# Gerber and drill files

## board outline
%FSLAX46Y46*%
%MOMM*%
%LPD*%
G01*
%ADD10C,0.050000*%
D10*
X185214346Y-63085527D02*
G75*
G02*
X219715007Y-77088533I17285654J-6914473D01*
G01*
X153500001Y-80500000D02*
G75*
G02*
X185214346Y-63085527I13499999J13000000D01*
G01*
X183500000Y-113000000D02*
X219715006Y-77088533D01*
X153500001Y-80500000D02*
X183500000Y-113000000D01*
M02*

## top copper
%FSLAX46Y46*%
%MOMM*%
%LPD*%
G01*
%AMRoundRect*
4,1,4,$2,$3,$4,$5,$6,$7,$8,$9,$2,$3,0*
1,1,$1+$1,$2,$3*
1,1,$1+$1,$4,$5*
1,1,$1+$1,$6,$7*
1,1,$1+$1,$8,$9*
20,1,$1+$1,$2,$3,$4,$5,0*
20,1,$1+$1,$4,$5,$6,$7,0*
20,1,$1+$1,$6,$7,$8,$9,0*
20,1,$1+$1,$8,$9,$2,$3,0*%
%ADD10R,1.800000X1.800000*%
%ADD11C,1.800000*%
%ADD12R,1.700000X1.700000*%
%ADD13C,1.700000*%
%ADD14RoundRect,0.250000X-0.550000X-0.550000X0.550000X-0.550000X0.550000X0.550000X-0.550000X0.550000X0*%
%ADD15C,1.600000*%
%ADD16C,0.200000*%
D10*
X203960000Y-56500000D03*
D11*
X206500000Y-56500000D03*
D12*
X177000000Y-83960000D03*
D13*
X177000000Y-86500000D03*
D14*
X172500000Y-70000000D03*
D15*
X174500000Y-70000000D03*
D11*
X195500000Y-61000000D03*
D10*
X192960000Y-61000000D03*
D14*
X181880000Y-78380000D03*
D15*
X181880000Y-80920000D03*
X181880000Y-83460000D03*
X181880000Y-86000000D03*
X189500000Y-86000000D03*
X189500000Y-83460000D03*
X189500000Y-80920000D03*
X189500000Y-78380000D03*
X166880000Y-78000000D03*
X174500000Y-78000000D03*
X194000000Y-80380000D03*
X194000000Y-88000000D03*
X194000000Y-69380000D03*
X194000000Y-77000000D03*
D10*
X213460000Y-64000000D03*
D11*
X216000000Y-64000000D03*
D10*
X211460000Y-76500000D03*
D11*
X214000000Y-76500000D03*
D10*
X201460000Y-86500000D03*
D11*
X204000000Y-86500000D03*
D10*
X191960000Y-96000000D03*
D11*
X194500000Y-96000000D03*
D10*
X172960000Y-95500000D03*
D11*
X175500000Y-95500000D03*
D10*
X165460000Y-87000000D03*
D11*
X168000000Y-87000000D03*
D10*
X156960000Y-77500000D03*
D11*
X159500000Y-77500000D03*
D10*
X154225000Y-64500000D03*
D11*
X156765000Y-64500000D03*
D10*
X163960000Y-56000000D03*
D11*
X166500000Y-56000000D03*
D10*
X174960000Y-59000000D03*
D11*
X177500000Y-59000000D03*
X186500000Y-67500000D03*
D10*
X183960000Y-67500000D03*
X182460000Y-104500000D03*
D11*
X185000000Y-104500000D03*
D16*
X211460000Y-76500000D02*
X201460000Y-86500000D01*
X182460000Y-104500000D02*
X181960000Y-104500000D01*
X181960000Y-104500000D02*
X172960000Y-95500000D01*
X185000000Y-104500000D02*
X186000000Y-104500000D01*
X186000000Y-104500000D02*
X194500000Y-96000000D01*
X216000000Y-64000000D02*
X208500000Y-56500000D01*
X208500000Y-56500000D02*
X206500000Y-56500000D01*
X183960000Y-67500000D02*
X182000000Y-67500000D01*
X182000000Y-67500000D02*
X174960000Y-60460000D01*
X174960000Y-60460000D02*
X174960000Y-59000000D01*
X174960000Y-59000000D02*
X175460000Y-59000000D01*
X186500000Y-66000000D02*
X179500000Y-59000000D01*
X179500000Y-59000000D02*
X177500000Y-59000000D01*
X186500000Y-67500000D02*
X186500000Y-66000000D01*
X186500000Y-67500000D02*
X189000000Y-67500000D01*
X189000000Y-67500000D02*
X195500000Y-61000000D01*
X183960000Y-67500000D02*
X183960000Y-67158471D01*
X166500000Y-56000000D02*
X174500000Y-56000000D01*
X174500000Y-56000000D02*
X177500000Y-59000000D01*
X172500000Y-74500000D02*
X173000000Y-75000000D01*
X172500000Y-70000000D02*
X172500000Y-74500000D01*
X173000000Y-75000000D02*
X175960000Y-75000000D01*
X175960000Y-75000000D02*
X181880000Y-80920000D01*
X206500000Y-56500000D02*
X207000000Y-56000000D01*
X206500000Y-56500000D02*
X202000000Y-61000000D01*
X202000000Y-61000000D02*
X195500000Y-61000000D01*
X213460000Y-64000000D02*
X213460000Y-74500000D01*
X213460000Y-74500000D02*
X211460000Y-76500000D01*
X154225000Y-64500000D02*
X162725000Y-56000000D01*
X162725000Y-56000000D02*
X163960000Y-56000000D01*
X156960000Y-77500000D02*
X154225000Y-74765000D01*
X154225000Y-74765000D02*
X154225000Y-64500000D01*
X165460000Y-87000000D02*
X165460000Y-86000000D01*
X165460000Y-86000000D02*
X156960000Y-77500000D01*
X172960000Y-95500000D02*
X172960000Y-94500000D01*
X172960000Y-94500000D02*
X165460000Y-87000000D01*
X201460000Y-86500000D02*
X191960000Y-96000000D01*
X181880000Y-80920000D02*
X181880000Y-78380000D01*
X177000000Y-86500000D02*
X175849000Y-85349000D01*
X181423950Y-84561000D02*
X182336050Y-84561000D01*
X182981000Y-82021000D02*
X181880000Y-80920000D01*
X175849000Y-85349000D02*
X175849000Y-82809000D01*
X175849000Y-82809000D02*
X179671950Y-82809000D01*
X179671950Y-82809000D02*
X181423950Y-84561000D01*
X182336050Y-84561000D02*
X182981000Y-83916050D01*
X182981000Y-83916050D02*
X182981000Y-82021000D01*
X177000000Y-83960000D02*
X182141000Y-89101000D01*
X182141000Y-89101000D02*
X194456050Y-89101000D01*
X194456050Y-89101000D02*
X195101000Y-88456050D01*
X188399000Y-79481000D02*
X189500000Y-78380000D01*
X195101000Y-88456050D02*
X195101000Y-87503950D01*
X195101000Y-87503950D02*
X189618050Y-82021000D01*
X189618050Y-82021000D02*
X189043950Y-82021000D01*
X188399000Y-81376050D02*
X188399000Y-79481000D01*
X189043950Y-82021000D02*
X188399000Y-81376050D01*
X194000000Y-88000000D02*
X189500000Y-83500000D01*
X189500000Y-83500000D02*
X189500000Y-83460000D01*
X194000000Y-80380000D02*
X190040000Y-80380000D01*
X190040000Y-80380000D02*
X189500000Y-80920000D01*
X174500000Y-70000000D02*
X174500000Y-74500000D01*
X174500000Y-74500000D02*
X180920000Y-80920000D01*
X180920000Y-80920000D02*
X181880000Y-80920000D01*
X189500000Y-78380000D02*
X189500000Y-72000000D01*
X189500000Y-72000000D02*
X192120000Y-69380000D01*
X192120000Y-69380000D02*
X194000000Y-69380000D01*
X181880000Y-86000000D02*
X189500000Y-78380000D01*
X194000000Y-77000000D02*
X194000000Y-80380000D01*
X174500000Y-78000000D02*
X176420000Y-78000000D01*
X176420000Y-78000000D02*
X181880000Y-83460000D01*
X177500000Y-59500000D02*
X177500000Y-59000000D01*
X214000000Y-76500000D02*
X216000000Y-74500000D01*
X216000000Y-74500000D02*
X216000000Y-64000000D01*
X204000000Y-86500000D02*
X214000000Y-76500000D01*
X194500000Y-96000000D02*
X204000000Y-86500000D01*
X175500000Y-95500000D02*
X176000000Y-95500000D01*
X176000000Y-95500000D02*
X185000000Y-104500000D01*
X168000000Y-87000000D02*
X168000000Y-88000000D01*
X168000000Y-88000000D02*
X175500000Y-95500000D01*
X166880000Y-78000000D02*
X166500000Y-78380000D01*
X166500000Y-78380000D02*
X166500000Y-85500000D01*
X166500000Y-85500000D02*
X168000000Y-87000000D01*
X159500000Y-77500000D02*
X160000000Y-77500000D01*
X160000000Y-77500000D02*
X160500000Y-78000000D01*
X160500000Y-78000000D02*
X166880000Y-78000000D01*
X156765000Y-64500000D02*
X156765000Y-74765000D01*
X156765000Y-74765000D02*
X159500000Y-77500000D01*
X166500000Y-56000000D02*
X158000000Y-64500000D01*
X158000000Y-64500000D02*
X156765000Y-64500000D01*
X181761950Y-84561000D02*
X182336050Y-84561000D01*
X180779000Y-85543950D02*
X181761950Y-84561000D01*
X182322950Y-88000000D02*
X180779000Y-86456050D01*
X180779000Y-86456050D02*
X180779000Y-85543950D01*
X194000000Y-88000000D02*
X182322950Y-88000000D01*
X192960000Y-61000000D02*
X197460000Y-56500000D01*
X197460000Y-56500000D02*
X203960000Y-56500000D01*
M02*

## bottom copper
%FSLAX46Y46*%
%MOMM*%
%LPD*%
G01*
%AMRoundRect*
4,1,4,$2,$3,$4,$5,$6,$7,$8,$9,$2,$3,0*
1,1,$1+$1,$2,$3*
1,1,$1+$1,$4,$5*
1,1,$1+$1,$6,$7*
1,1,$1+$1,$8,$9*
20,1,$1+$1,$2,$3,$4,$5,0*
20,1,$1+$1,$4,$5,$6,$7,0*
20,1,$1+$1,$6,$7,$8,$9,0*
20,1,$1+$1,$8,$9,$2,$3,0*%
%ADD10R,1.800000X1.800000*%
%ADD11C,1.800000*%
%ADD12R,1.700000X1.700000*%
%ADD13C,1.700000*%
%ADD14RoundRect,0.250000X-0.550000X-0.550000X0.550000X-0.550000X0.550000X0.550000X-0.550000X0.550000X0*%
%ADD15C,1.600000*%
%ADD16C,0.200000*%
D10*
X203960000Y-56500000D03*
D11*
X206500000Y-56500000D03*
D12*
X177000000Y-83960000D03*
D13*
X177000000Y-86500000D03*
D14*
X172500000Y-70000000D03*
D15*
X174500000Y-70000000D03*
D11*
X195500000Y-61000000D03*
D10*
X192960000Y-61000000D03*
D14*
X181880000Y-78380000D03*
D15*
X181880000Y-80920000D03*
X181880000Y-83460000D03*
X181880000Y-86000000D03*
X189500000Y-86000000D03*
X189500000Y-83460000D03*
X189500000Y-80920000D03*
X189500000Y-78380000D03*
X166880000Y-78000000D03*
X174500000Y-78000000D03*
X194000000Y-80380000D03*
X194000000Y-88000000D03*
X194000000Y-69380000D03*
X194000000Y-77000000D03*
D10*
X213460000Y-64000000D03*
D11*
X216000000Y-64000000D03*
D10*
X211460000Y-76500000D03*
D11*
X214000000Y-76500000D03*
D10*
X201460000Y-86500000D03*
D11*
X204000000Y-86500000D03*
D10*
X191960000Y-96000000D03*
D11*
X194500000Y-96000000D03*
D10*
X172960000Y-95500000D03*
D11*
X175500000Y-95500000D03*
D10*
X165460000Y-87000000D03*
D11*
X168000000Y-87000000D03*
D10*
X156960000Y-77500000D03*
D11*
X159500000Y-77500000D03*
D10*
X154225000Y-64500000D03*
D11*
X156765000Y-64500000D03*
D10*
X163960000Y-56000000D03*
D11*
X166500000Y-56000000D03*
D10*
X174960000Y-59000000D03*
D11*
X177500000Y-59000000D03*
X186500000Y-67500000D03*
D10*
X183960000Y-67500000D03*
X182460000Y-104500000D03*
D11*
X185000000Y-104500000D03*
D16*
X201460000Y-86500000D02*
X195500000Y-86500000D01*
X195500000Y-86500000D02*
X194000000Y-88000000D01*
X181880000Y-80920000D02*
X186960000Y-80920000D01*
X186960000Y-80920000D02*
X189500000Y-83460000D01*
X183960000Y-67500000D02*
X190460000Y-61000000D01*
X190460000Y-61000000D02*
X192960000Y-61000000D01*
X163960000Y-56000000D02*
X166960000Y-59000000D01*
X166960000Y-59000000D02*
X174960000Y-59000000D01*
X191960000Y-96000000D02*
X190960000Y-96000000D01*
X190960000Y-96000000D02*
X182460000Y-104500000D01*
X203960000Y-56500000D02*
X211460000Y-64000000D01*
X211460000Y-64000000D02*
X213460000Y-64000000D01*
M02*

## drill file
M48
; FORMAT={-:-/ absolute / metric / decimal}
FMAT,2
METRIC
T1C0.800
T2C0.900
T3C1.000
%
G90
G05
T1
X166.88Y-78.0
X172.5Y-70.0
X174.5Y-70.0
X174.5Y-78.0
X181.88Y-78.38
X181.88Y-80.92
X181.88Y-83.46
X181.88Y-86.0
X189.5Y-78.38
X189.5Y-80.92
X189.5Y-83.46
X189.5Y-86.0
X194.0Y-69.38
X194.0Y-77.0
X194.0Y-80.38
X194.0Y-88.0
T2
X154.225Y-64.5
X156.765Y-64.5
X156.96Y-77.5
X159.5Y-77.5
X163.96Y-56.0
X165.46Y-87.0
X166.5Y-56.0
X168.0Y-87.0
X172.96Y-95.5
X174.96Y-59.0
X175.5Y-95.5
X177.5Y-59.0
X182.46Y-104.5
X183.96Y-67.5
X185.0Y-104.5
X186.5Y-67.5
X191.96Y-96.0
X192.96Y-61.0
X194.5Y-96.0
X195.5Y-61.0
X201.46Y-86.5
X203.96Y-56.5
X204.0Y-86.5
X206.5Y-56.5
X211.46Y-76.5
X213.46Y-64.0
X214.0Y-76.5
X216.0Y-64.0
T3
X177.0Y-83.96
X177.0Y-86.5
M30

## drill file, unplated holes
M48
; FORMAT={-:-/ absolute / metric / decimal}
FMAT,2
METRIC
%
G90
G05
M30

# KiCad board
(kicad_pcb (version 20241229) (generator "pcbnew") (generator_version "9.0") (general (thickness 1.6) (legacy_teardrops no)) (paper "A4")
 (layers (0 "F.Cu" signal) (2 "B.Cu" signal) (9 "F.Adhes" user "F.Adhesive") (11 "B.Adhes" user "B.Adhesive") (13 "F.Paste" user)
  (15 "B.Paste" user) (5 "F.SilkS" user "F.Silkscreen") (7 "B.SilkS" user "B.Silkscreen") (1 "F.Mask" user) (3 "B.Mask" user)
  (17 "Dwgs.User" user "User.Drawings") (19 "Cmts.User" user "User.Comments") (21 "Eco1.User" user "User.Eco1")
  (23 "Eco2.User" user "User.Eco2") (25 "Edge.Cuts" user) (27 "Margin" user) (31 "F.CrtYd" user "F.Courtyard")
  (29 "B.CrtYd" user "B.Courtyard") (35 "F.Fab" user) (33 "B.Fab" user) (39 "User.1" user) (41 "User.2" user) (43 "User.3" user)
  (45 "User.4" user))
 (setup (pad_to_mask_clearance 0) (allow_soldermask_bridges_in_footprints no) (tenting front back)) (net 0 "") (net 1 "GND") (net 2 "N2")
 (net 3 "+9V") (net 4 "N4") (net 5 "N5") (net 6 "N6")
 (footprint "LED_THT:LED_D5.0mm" (layer "F.Cu") (at 183.96 67.5)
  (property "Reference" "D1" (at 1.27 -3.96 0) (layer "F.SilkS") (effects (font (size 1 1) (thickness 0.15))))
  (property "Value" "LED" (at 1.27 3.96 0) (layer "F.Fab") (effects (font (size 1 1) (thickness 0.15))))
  (pad "1" thru_hole rect (at 0 0) (size 1.8 1.8) (drill 0.9) (layers "*.Cu" "*.Mask") (remove_unused_layers no) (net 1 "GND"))
  (pad "2" thru_hole circle (at 2.54 0) (size 1.8 1.8) (drill 0.9) (layers "*.Cu" "*.Mask") (remove_unused_layers no) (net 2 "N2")))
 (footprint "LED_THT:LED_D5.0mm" (layer "F.Cu") (at 192.96 61)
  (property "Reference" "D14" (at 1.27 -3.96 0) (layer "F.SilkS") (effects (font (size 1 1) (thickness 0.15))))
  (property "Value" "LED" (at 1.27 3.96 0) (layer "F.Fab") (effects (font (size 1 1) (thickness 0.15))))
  (pad "1" thru_hole rect (at 0 0) (size 1.8 1.8) (drill 0.9) (layers "*.Cu" "*.Mask") (remove_unused_layers no) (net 1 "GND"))
  (pad "2" thru_hole circle (at 2.54 0) (size 1.8 1.8) (drill 0.9) (layers "*.Cu" "*.Mask") (remove_unused_layers no) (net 2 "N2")))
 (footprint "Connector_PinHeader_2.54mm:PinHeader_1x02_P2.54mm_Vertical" (layer "F.Cu") (at 177 83.96)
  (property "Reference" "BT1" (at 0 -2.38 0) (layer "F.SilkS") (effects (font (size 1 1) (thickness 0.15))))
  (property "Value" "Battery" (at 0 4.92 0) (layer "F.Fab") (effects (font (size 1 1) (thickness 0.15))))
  (pad "1" thru_hole rect (at 0 0) (size 1.7 1.7) (drill 1) (layers "*.Cu" "*.Mask") (remove_unused_layers no) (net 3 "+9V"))
  (pad "2" thru_hole circle (at 0 2.54) (size 1.7 1.7) (drill 1) (layers "*.Cu" "*.Mask") (remove_unused_layers no) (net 1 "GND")))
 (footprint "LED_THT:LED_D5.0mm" (layer "F.Cu") (at 203.96 56.5)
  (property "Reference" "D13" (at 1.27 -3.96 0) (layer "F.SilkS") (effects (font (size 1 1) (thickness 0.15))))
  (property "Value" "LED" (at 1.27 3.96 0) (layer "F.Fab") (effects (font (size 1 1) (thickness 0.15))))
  (pad "1" thru_hole rect (at 0 0) (size 1.8 1.8) (drill 0.9) (layers "*.Cu" "*.Mask") (remove_unused_layers no) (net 1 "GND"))
  (pad "2" thru_hole circle (at 2.54 0) (size 1.8 1.8) (drill 0.9) (layers "*.Cu" "*.Mask") (remove_unused_layers no) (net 2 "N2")))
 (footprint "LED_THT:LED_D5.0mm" (layer "F.Cu") (at 154.225 64.5)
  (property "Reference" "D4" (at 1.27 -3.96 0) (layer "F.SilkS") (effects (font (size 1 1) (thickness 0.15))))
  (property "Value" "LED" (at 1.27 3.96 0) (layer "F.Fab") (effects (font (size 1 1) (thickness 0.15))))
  (pad "1" thru_hole rect (at 0 0) (size 1.8 1.8) (drill 0.9) (layers "*.Cu" "*.Mask") (remove_unused_layers no) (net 1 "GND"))
  (pad "2" thru_hole circle (at 2.54 0) (size 1.8 1.8) (drill 0.9) (layers "*.Cu" "*.Mask") (remove_unused_layers no) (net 2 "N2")))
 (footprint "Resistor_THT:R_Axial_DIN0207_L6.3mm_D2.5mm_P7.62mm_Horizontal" (layer "F.Cu") (at 166.88 78)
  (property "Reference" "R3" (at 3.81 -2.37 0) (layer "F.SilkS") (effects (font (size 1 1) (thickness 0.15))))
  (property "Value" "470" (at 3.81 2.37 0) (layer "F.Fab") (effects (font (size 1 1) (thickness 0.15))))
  (pad "1" thru_hole circle (at 0 0) (size 1.6 1.6) (drill 0.8) (layers "*.Cu" "*.Mask") (remove_unused_layers no) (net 2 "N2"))
  (pad "2" thru_hole circle (at 7.62 0) (size 1.6 1.6) (drill 0.8) (layers "*.Cu" "*.Mask") (remove_unused_layers no) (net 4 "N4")))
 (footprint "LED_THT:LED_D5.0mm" (layer "F.Cu") (at 172.96 95.5)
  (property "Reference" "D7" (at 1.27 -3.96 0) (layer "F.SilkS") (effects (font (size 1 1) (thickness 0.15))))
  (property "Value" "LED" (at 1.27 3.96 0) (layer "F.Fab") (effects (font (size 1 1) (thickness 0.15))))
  (pad "1" thru_hole rect (at 0 0) (size 1.8 1.8) (drill 0.9) (layers "*.Cu" "*.Mask") (remove_unused_layers no) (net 1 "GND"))
  (pad "2" thru_hole circle (at 2.54 0) (size 1.8 1.8) (drill 0.9) (layers "*.Cu" "*.Mask") (remove_unused_layers no) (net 2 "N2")))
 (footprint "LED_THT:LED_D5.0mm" (layer "F.Cu") (at 191.96 96)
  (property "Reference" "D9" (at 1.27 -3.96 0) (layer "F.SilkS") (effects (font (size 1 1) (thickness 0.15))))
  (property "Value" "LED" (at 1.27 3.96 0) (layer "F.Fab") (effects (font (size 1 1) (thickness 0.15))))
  (pad "1" thru_hole rect (at 0 0) (size 1.8 1.8) (drill 0.9) (layers "*.Cu" "*.Mask") (remove_unused_layers no) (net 1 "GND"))
  (pad "2" thru_hole circle (at 2.54 0) (size 1.8 1.8) (drill 0.9) (layers "*.Cu" "*.Mask") (remove_unused_layers no) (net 2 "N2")))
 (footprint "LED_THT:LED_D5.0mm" (layer "F.Cu") (at 213.46 64)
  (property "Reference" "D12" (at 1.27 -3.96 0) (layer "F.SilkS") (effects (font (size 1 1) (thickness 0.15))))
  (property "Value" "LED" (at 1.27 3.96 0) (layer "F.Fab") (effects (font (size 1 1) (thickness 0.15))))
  (pad "1" thru_hole rect (at 0 0) (size 1.8 1.8) (drill 0.9) (layers "*.Cu" "*.Mask") (remove_unused_layers no) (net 1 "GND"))
  (pad "2" thru_hole circle (at 2.54 0) (size 1.8 1.8) (drill 0.9) (layers "*.Cu" "*.Mask") (remove_unused_layers no) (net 2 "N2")))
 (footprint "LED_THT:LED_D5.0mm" (layer "F.Cu") (at 201.46 86.5)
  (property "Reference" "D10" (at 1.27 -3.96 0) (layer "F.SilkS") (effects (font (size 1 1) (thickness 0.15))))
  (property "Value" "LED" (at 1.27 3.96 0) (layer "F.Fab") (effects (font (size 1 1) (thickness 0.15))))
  (pad "1" thru_hole rect (at 0 0) (size 1.8 1.8) (drill 0.9) (layers "*.Cu" "*.Mask") (remove_unused_layers no) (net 1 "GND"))
  (pad "2" thru_hole circle (at 2.54 0) (size 1.8 1.8) (drill 0.9) (layers "*.Cu" "*.Mask") (remove_unused_layers no) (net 2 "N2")))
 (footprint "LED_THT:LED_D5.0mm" (layer "F.Cu") (at 182.46 104.5)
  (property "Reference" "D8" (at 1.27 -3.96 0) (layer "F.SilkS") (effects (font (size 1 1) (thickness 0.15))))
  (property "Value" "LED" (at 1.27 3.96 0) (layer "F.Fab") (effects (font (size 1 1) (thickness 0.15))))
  (pad "1" thru_hole rect (at 0 0) (size 1.8 1.8) (drill 0.9) (layers "*.Cu" "*.Mask") (remove_unused_layers no) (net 1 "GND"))
  (pad "2" thru_hole circle (at 2.54 0) (size 1.8 1.8) (drill 0.9) (layers "*.Cu" "*.Mask") (remove_unused_layers no) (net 2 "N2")))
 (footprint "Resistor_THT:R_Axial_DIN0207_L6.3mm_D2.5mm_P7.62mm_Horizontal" (layer "F.Cu") (at 194 69.38 -90)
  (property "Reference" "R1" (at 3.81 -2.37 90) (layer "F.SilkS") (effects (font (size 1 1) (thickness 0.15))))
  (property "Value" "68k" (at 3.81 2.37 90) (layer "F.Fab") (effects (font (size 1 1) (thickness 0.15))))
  (pad "1" thru_hole circle (at 0 0 270) (size 1.6 1.6) (drill 0.8) (layers "*.Cu" "*.Mask") (remove_unused_layers no) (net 3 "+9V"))
  (pad "2" thru_hole circle (at 7.62 0 270) (size 1.6 1.6) (drill 0.8) (layers "*.Cu" "*.Mask") (remove_unused_layers no) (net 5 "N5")))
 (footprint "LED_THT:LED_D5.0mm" (layer "F.Cu") (at 174.96 59)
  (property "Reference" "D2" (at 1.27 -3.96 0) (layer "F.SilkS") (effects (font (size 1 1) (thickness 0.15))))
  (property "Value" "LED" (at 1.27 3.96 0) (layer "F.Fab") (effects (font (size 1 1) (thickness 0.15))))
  (pad "1" thru_hole rect (at 0 0) (size 1.8 1.8) (drill 0.9) (layers "*.Cu" "*.Mask") (remove_unused_layers no) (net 1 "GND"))
  (pad "2" thru_hole circle (at 2.54 0) (size 1.8 1.8) (drill 0.9) (layers "*.Cu" "*.Mask") (remove_unused_layers no) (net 2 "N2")))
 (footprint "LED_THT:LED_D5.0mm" (layer "F.Cu") (at 211.46 76.5)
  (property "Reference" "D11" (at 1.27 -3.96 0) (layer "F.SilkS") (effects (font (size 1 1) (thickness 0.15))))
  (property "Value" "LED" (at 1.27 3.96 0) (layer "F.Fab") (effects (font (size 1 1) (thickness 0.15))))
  (pad "1" thru_hole rect (at 0 0) (size 1.8 1.8) (drill 0.9) (layers "*.Cu" "*.Mask") (remove_unused_layers no) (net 1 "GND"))
  (pad "2" thru_hole circle (at 2.54 0) (size 1.8 1.8) (drill 0.9) (layers "*.Cu" "*.Mask") (remove_unused_layers no) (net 2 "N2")))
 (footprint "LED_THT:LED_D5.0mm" (layer "F.Cu") (at 165.46 87)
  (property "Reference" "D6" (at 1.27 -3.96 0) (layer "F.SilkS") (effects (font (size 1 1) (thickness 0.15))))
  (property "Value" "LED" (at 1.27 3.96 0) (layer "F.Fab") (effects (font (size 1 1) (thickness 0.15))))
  (pad "1" thru_hole rect (at 0 0) (size 1.8 1.8) (drill 0.9) (layers "*.Cu" "*.Mask") (remove_unused_layers no) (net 1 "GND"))
  (pad "2" thru_hole circle (at 2.54 0) (size 1.8 1.8) (drill 0.9) (layers "*.Cu" "*.Mask") (remove_unused_layers no) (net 2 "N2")))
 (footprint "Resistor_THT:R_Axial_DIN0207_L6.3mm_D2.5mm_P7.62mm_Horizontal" (layer "F.Cu") (at 194 80.38 -90)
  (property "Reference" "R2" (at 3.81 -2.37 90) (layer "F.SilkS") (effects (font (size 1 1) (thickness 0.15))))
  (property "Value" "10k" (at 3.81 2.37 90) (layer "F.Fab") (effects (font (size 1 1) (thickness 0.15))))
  (pad "1" thru_hole circle (at 0 0 270) (size 1.6 1.6) (drill 0.8) (layers "*.Cu" "*.Mask") (remove_unused_layers no) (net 5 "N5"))
  (pad "2" thru_hole circle (at 7.62 0 270) (size 1.6 1.6) (drill 0.8) (layers "*.Cu" "*.Mask") (remove_unused_layers no) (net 1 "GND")))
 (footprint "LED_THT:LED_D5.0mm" (layer "F.Cu") (at 156.96 77.5)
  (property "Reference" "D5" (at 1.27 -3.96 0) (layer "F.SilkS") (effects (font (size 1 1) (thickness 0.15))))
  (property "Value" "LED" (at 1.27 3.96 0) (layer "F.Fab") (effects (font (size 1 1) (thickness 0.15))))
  (pad "1" thru_hole rect (at 0 0) (size 1.8 1.8) (drill 0.9) (layers "*.Cu" "*.Mask") (remove_unused_layers no) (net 1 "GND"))
  (pad "2" thru_hole circle (at 2.54 0) (size 1.8 1.8) (drill 0.9) (layers "*.Cu" "*.Mask") (remove_unused_layers no) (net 2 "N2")))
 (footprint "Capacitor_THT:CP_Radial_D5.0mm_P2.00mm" (layer "F.Cu") (at 172.5 70)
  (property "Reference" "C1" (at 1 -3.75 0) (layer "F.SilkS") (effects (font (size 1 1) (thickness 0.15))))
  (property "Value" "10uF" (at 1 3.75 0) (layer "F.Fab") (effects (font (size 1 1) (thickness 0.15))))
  (pad "1" thru_hole roundrect (at 0 0) (size 1.6 1.6) (drill 0.8) (layers "*.Cu" "*.Mask") (remove_unused_layers no)
   (roundrect_rratio 0.15625) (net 1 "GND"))
  (pad "2" thru_hole circle (at 2 0) (size 1.6 1.6) (drill 0.8) (layers "*.Cu" "*.Mask") (remove_unused_layers no) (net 1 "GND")))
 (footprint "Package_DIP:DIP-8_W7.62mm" (layer "F.Cu") (at 181.88 78.38)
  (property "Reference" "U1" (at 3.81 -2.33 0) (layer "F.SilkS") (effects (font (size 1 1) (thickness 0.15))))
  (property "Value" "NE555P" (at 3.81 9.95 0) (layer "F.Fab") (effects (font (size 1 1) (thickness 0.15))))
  (pad "1" thru_hole roundrect (at 0 0) (size 1.6 1.6) (drill 0.8) (layers "*.Cu" "*.Mask") (remove_unused_layers no)
   (roundrect_rratio 0.15625) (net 1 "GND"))
  (pad "2" thru_hole circle (at 0 2.54) (size 1.6 1.6) (drill 0.8) (layers "*.Cu" "*.Mask") (remove_unused_layers no) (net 1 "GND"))
  (pad "3" thru_hole circle (at 0 5.08) (size 1.6 1.6) (drill 0.8) (layers "*.Cu" "*.Mask") (remove_unused_layers no) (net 4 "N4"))
  (pad "4" thru_hole circle (at 0 7.62) (size 1.6 1.6) (drill 0.8) (layers "*.Cu" "*.Mask") (remove_unused_layers no) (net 3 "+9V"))
  (pad "5" thru_hole circle (at 7.62 7.62) (size 1.6 1.6) (drill 0.8) (layers "*.Cu" "*.Mask") (remove_unused_layers no) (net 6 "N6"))
  (pad "6" thru_hole circle (at 7.62 5.08) (size 1.6 1.6) (drill 0.8) (layers "*.Cu" "*.Mask") (remove_unused_layers no) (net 1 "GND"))
  (pad "7" thru_hole circle (at 7.62 2.54) (size 1.6 1.6) (drill 0.8) (layers "*.Cu" "*.Mask") (remove_unused_layers no) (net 5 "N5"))
  (pad "8" thru_hole circle (at 7.62 0) (size 1.6 1.6) (drill 0.8) (layers "*.Cu" "*.Mask") (remove_unused_layers no) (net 3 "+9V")))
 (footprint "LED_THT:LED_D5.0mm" (layer "F.Cu") (at 163.96 56)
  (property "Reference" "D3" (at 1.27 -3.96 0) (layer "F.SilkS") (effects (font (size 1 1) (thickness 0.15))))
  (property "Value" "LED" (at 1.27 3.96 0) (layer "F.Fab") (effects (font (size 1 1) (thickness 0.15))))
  (pad "1" thru_hole rect (at 0 0) (size 1.8 1.8) (drill 0.9) (layers "*.Cu" "*.Mask") (remove_unused_layers no) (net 1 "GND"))
  (pad "2" thru_hole circle (at 2.54 0) (size 1.8 1.8) (drill 0.9) (layers "*.Cu" "*.Mask") (remove_unused_layers no) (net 2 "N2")))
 (gr_line (start 153.500001 80.5) (end 183.5 113) (stroke (width 0.05) (type default)) (layer "Edge.Cuts"))
 (gr_arc (start 185.214346 63.085527) (mid 209.501592 52.74945) (end 219.715008 77.088533) (stroke (width 0.05) (type default))
  (layer "Edge.Cuts"))
 (gr_arc (start 153.500001 80.5) (mid 157.979344 51.072044) (end 185.214346 63.085527) (stroke (width 0.05) (type default))
  (layer "Edge.Cuts"))
 (gr_line (start 183.5 113) (end 219.715006 77.088533) (stroke (width 0.05) (type default)) (layer "Edge.Cuts"))
 (segment (start 181.88 86) (end 189.5 78.38) (width 0.2) (layer "F.Cu") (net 3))
 (segment (start 189.5 72) (end 192.12 69.38) (width 0.2) (layer "F.Cu") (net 3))
 (segment (start 188.399 79.481) (end 189.5 78.38) (width 0.2) (layer "F.Cu") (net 3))
 (segment (start 192.12 69.38) (end 194 69.38) (width 0.2) (layer "F.Cu") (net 3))
 (segment (start 177 83.96) (end 182.141 89.101) (width 0.2) (layer "F.Cu") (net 3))
 (segment (start 189.5 78.38) (end 189.5 72) (width 0.2) (layer "F.Cu") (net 3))
 (segment (start 189.61805 82.021) (end 189.04395 82.021) (width 0.2) (layer "F.Cu") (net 3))
 (segment (start 194.45605 89.101) (end 195.101 88.45605) (width 0.2) (layer "F.Cu") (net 3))
 (segment (start 188.399 81.37605) (end 188.399 79.481) (width 0.2) (layer "F.Cu") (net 3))
 (segment (start 195.101 87.50395) (end 189.61805 82.021) (width 0.2) (layer "F.Cu") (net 3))
 (segment (start 195.101 88.45605) (end 195.101 87.50395) (width 0.2) (layer "F.Cu") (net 3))
 (segment (start 182.141 89.101) (end 194.45605 89.101) (width 0.2) (layer "F.Cu") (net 3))
 (segment (start 189.04395 82.021) (end 188.399 81.37605) (width 0.2) (layer "F.Cu") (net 3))
 (segment (start 213.46 74.5) (end 211.46 76.5) (width 0.2) (layer "F.Cu") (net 1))
 (segment (start 172.5 74.5) (end 173 75) (width 0.2) (layer "F.Cu") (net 1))
 (segment (start 181.88 80.92) (end 181.88 78.38) (width 0.2) (layer "F.Cu") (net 1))
 (segment (start 182.46 104.5) (end 181.96 104.5) (width 0.2) (layer "F.Cu") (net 1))
 (segment (start 180.779 85.54395) (end 181.76195 84.561) (width 0.2) (layer "F.Cu") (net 1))
 (segment (start 181.42395 84.561) (end 182.33605 84.561) (width 0.2) (layer "F.Cu") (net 1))
 (segment (start 213.46 64) (end 213.46 74.5) (width 0.2) (layer "F.Cu") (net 1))
 (segment (start 182.32295 88) (end 180.779 86.45605) (width 0.2) (layer "F.Cu") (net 1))
 (segment (start 175.849 82.809) (end 179.67195 82.809) (width 0.2) (layer "F.Cu") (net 1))
 (segment (start 192.96 61) (end 197.46 56.5) (width 0.2) (layer "F.Cu") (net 1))
 (segment (start 181.76195 84.561) (end 182.33605 84.561) (width 0.2) (layer "F.Cu") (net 1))
 (segment (start 173 75) (end 175.96 75) (width 0.2) (layer "F.Cu") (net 1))
 (segment (start 194 88) (end 182.32295 88) (width 0.2) (layer "F.Cu") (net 1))
 (segment (start 154.225 64.5) (end 162.725 56) (width 0.2) (layer "F.Cu") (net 1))
 (segment (start 174.5 74.5) (end 180.92 80.92) (width 0.2) (layer "F.Cu") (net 1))
 (segment (start 175.96 75) (end 181.88 80.92) (width 0.2) (layer "F.Cu") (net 1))
 (segment (start 172.96 94.5) (end 165.46 87) (width 0.2) (layer "F.Cu") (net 1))
 (segment (start 182 67.5) (end 174.96 60.46) (width 0.2) (layer "F.Cu") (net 1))
 (segment (start 174.5 70) (end 174.5 74.5) (width 0.2) (layer "F.Cu") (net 1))
 (segment (start 180.92 80.92) (end 181.88 80.92) (width 0.2) (layer "F.Cu") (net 1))
 (segment (start 183.96 67.5) (end 183.96 67.158471) (width 0.2) (layer "F.Cu") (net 1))
 (segment (start 180.779 86.45605) (end 180.779 85.54395) (width 0.2) (layer "F.Cu") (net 1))
 (segment (start 182.981 82.021) (end 181.88 80.92) (width 0.2) (layer "F.Cu") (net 1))
 (segment (start 175.849 85.349) (end 175.849 82.809) (width 0.2) (layer "F.Cu") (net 1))
 (segment (start 177 86.5) (end 175.849 85.349) (width 0.2) (layer "F.Cu") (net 1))
 (segment (start 201.46 86.5) (end 191.96 96) (width 0.2) (layer "F.Cu") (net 1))
 (segment (start 154.225 74.765) (end 154.225 64.5) (width 0.2) (layer "F.Cu") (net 1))
 (segment (start 197.46 56.5) (end 203.96 56.5) (width 0.2) (layer "F.Cu") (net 1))
 (segment (start 174.96 60.46) (end 174.96 59) (width 0.2) (layer "F.Cu") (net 1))
 (segment (start 165.46 87) (end 165.46 86) (width 0.2) (layer "F.Cu") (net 1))
 (segment (start 156.96 77.5) (end 154.225 74.765) (width 0.2) (layer "F.Cu") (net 1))
 (segment (start 194 88) (end 189.5 83.5) (width 0.2) (layer "F.Cu") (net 1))
 (segment (start 189.5 83.5) (end 189.5 83.46) (width 0.2) (layer "F.Cu") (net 1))
 (segment (start 211.46 76.5) (end 201.46 86.5) (width 0.2) (layer "F.Cu") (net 1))
 (segment (start 182.981 83.91605) (end 182.981 82.021) (width 0.2) (layer "F.Cu") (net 1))
 (segment (start 182.33605 84.561) (end 182.981 83.91605) (width 0.2) (layer "F.Cu") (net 1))
 (segment (start 183.96 67.5) (end 182 67.5) (width 0.2) (layer "F.Cu") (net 1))
 (segment (start 162.725 56) (end 163.96 56) (width 0.2) (layer "F.Cu") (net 1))
 (segment (start 172.5 70) (end 172.5 74.5) (width 0.2) (layer "F.Cu") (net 1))
 (segment (start 174.96 59) (end 175.46 59) (width 0.2) (layer "F.Cu") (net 1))
 (segment (start 179.67195 82.809) (end 181.42395 84.561) (width 0.2) (layer "F.Cu") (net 1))
 (segment (start 165.46 86) (end 156.96 77.5) (width 0.2) (layer "F.Cu") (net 1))
 (segment (start 181.96 104.5) (end 172.96 95.5) (width 0.2) (layer "F.Cu") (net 1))
 (segment (start 172.96 95.5) (end 172.96 94.5) (width 0.2) (layer "F.Cu") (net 1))
 (segment (start 183.96 67.5) (end 190.46 61) (width 0.2) (layer "B.Cu") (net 1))
 (segment (start 190.46 61) (end 192.96 61) (width 0.2) (layer "B.Cu") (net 1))
 (segment (start 191.96 96) (end 190.96 96) (width 0.2) (layer "B.Cu") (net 1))
 (segment (start 195.5 86.5) (end 194 88) (width 0.2) (layer "B.Cu") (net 1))
 (segment (start 163.96 56) (end 166.96 59) (width 0.2) (layer "B.Cu") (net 1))
 (segment (start 203.96 56.5) (end 211.46 64) (width 0.2) (layer "B.Cu") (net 1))
 (segment (start 211.46 64) (end 213.46 64) (width 0.2) (layer "B.Cu") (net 1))
 (segment (start 186.96 80.92) (end 189.5 83.46) (width 0.2) (layer "B.Cu") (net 1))
 (segment (start 190.96 96) (end 182.46 104.5) (width 0.2) (layer "B.Cu") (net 1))
 (segment (start 201.46 86.5) (end 195.5 86.5) (width 0.2) (layer "B.Cu") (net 1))
 (segment (start 181.88 80.92) (end 186.96 80.92) (width 0.2) (layer "B.Cu") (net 1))
 (segment (start 166.96 59) (end 174.96 59) (width 0.2) (layer "B.Cu") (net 1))
 (segment (start 160 77.5) (end 160.5 78) (width 0.2) (layer "F.Cu") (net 2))
 (segment (start 194.5 96) (end 204 86.5) (width 0.2) (layer "F.Cu") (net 2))
 (segment (start 185 104.5) (end 186 104.5) (width 0.2) (layer "F.Cu") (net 2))
 (segment (start 168 88) (end 175.5 95.5) (width 0.2) (layer "F.Cu") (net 2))
 (segment (start 158 64.5) (end 156.765 64.5) (width 0.2) (layer "F.Cu") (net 2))
 (segment (start 202 61) (end 195.5 61) (width 0.2) (layer "F.Cu") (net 2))
 (segment (start 206.5 56.5) (end 207 56) (width 0.2) (layer "F.Cu") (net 2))
 (segment (start 214 76.5) (end 216 74.5) (width 0.2) (layer "F.Cu") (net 2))
 (segment (start 186.5 67.5) (end 186.5 66) (width 0.2) (layer "F.Cu") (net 2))
 (segment (start 189 67.5) (end 195.5 61) (width 0.2) (layer "F.Cu") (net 2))
 (segment (start 166.5 56) (end 158 64.5) (width 0.2) (layer "F.Cu") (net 2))
 (segment (start 159.5 77.5) (end 160 77.5) (width 0.2) (layer "F.Cu") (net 2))
 (segment (start 166.5 85.5) (end 168 87) (width 0.2) (layer "F.Cu") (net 2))
 (segment (start 166.5 56) (end 174.5 56) (width 0.2) (layer "F.Cu") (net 2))
 (segment (start 166.5 78.38) (end 166.5 85.5) (width 0.2) (layer "F.Cu") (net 2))
 (segment (start 216 74.5) (end 216 64) (width 0.2) (layer "F.Cu") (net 2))
 (segment (start 208.5 56.5) (end 206.5 56.5) (width 0.2) (layer "F.Cu") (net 2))
 (segment (start 156.765 74.765) (end 159.5 77.5) (width 0.2) (layer "F.Cu") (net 2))
 (segment (start 168 87) (end 168 88) (width 0.2) (layer "F.Cu") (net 2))
 (segment (start 160.5 78) (end 166.88 78) (width 0.2) (layer "F.Cu") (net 2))
 (segment (start 175.5 95.5) (end 176 95.5) (width 0.2) (layer "F.Cu") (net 2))
 (segment (start 186.5 66) (end 179.5 59) (width 0.2) (layer "F.Cu") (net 2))
 (segment (start 156.765 64.5) (end 156.765 74.765) (width 0.2) (layer "F.Cu") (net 2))
 (segment (start 177.5 59.5) (end 177.5 59) (width 0.2) (layer "F.Cu") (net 2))
 (segment (start 166.88 78) (end 166.5 78.38) (width 0.2) (layer "F.Cu") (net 2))
 (segment (start 174.5 56) (end 177.5 59) (width 0.2) (layer "F.Cu") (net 2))
 (segment (start 186 104.5) (end 194.5 96) (width 0.2) (layer "F.Cu") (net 2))
 (segment (start 186.5 67.5) (end 189 67.5) (width 0.2) (layer "F.Cu") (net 2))
 (segment (start 216 64) (end 208.5 56.5) (width 0.2) (layer "F.Cu") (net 2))
 (segment (start 206.5 56.5) (end 202 61) (width 0.2) (layer "F.Cu") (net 2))
 (segment (start 204 86.5) (end 214 76.5) (width 0.2) (layer "F.Cu") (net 2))
 (segment (start 176 95.5) (end 185 104.5) (width 0.2) (layer "F.Cu") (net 2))
 (segment (start 179.5 59) (end 177.5 59) (width 0.2) (layer "F.Cu") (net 2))
 (segment (start 176.42 78) (end 181.88 83.46) (width 0.2) (layer "F.Cu") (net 4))
 (segment (start 174.5 78) (end 176.42 78) (width 0.2) (layer "F.Cu") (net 4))
 (segment (start 190.04 80.38) (end 189.5 80.92) (width 0.2) (layer "F.Cu") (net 5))
 (segment (start 194 77) (end 194 80.38) (width 0.2) (layer "F.Cu") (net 5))
 (segment (start 194 80.38) (end 190.04 80.38) (width 0.2) (layer "F.Cu") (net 5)))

